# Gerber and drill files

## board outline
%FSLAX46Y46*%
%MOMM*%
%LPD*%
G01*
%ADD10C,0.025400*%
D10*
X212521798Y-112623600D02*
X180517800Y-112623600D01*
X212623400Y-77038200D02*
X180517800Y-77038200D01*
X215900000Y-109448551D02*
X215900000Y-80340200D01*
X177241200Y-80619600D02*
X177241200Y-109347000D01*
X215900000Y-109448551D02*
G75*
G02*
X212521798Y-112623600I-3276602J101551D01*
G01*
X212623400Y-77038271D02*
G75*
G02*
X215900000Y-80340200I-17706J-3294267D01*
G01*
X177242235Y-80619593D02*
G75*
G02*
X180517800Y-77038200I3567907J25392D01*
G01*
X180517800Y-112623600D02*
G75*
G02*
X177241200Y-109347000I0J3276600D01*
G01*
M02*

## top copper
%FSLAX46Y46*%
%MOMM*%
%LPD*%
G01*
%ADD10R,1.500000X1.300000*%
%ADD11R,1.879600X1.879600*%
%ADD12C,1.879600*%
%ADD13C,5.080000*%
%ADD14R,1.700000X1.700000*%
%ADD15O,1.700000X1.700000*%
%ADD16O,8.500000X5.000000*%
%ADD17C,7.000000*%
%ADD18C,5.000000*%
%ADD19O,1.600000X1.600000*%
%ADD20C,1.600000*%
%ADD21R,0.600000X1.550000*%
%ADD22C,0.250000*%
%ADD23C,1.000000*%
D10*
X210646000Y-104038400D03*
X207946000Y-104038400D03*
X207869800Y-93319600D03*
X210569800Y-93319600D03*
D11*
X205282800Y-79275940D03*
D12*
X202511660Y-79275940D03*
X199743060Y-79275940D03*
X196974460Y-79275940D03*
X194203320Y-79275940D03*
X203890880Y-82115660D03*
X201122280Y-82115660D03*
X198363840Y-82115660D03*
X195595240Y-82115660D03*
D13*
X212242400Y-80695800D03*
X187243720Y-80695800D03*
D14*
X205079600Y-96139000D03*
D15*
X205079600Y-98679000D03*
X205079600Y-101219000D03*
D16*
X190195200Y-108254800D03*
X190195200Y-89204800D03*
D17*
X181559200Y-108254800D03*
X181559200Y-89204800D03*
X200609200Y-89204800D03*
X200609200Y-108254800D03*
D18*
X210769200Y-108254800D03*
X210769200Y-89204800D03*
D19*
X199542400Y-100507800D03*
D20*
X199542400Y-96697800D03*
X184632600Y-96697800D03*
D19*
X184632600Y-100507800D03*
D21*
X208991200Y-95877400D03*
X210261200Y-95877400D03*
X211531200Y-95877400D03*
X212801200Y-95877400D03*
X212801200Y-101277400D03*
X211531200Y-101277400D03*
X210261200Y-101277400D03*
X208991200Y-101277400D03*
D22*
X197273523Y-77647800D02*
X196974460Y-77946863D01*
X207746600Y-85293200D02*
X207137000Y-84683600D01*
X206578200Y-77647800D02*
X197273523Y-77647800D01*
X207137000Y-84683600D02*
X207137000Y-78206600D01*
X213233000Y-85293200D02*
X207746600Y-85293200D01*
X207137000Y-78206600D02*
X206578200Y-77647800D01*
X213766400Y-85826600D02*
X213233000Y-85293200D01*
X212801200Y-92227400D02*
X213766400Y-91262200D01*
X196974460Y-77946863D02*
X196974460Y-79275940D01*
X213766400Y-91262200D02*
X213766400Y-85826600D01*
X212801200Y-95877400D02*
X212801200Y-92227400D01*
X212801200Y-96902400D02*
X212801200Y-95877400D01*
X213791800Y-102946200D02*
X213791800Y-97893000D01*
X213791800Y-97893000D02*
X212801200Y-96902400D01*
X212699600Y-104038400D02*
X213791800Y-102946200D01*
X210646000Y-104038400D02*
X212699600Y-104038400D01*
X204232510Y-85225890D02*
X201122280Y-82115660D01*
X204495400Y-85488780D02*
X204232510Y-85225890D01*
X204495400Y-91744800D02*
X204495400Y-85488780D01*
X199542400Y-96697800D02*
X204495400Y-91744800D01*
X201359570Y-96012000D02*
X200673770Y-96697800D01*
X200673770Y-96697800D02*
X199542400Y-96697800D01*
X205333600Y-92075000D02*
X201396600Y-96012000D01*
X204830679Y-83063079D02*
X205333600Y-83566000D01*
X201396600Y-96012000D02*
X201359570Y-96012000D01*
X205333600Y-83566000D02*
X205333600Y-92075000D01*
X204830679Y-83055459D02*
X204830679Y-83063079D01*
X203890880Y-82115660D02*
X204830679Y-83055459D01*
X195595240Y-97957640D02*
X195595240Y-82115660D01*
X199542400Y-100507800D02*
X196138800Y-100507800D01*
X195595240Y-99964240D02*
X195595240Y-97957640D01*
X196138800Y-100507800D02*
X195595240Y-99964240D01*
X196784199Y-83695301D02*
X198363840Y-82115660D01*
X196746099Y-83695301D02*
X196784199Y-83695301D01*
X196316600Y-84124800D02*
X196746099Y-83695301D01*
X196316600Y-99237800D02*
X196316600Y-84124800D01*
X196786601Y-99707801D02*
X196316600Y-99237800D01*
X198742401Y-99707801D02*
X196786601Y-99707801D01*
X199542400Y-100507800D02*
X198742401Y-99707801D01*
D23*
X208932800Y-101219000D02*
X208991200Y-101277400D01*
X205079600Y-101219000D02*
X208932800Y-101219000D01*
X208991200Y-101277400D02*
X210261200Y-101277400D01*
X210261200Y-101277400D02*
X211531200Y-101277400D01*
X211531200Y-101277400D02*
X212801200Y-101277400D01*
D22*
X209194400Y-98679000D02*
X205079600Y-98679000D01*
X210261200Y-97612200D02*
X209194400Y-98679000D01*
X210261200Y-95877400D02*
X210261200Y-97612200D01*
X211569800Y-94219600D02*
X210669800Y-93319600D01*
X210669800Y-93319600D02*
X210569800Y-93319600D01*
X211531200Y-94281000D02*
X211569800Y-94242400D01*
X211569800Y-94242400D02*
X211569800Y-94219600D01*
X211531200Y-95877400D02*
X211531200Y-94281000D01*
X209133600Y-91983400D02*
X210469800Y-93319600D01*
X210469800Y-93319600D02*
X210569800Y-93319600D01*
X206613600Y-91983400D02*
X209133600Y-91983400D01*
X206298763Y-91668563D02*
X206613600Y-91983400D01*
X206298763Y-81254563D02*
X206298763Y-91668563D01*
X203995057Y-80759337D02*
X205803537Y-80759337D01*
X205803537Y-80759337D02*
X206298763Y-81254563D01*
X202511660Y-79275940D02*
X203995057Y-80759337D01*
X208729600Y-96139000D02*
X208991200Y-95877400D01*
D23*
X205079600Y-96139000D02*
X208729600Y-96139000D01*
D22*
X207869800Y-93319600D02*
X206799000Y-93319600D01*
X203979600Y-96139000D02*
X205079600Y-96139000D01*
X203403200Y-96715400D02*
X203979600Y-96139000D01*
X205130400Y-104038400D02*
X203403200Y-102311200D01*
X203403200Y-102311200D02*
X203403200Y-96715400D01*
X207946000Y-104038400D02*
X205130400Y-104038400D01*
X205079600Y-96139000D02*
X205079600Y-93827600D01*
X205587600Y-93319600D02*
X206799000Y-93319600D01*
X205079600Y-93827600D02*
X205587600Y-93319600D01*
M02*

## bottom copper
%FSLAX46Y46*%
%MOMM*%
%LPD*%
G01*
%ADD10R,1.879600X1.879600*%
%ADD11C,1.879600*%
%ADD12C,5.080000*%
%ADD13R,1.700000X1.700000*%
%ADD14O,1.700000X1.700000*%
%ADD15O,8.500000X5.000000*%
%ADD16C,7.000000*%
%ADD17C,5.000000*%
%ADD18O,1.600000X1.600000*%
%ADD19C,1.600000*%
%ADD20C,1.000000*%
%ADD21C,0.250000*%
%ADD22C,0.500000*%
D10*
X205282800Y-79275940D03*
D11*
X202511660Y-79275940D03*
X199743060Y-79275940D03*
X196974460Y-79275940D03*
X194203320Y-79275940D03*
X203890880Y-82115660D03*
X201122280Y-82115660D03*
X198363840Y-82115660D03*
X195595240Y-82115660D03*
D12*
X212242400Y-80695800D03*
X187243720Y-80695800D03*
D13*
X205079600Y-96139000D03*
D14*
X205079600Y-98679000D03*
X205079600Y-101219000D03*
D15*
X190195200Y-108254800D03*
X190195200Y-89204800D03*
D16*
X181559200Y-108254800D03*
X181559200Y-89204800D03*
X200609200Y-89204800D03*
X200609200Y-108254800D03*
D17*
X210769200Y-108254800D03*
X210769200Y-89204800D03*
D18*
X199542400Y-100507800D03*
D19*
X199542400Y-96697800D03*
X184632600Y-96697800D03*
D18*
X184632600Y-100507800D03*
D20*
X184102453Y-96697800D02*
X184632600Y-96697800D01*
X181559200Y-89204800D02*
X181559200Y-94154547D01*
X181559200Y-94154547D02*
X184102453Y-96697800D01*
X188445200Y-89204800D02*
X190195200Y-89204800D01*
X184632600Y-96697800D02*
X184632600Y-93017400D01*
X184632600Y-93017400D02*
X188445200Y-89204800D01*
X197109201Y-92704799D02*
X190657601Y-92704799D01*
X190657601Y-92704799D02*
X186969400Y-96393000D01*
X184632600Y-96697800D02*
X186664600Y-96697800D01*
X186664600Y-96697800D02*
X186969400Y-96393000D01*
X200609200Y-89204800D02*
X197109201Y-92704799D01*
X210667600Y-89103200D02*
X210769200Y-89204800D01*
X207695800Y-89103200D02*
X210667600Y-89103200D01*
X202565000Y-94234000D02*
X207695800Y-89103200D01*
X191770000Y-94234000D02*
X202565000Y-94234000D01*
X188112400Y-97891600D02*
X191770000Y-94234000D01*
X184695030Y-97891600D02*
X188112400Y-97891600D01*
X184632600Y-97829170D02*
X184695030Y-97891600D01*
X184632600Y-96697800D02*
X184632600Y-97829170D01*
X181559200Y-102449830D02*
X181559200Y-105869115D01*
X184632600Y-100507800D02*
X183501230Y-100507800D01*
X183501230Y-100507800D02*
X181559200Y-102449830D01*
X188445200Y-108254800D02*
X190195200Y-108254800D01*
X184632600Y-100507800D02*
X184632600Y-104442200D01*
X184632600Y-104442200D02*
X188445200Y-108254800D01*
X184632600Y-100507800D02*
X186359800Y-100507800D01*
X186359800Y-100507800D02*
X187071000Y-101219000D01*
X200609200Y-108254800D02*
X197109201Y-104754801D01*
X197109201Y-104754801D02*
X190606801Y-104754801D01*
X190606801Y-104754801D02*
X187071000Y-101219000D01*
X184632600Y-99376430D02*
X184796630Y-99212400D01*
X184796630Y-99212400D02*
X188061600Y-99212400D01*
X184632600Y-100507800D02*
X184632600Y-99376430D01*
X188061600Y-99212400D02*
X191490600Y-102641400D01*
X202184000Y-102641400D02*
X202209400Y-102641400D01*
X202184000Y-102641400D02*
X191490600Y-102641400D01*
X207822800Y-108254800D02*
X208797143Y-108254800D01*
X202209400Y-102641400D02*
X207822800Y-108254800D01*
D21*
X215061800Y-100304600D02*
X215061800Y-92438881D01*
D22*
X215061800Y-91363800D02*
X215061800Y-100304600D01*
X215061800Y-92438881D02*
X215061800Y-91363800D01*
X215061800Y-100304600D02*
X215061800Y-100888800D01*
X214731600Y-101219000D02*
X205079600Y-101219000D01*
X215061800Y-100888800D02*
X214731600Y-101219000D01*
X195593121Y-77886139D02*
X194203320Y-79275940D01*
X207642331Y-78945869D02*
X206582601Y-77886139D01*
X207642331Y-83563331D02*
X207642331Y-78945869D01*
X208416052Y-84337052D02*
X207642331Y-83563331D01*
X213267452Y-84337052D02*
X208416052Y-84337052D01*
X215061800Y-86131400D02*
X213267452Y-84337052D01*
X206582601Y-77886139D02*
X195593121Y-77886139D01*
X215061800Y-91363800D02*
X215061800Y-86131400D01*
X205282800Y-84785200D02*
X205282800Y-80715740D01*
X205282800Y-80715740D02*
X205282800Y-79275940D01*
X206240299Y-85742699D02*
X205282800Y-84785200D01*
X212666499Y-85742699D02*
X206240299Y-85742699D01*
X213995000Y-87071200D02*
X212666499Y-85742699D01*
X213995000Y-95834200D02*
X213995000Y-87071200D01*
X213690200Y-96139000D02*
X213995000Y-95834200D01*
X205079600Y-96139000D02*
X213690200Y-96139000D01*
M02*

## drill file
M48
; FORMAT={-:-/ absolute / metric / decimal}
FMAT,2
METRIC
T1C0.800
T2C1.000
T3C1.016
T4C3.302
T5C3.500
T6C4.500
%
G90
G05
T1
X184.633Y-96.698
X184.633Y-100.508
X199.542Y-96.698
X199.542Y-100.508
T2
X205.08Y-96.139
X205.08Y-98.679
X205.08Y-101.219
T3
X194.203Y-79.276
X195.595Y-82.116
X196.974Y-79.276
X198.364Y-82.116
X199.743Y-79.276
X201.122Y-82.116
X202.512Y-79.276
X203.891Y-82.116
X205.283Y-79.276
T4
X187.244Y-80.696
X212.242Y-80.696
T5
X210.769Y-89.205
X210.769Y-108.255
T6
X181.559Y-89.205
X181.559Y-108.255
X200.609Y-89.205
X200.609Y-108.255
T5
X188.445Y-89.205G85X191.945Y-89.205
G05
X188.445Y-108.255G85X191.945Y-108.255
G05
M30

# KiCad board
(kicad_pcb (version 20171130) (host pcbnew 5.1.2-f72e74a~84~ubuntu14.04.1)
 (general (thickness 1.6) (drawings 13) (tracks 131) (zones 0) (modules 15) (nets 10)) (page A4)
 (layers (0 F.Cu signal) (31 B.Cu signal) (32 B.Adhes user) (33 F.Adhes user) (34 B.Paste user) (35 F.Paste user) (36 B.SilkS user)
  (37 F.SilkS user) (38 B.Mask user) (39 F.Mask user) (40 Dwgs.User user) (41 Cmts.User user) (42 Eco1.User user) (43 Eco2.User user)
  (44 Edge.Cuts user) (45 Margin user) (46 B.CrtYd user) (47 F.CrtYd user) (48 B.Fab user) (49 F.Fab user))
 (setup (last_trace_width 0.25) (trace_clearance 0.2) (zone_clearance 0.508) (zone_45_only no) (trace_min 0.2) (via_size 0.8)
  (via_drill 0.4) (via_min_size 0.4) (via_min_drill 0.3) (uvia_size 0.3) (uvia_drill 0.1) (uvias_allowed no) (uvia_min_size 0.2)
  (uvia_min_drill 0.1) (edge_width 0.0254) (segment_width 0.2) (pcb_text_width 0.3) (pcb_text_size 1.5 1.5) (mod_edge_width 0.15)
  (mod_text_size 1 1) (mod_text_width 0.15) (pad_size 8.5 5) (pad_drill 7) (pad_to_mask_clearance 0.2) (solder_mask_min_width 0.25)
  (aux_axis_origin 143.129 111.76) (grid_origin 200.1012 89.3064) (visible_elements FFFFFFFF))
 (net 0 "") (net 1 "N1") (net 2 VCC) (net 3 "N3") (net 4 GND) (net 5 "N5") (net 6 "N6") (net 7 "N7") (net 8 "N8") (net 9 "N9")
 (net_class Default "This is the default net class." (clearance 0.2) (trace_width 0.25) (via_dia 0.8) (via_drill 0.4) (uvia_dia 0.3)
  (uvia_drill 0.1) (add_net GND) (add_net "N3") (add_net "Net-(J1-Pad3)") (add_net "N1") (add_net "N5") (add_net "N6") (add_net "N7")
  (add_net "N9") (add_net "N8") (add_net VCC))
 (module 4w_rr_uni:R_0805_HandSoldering (layer F.Cu) (at 209.296 104.0384)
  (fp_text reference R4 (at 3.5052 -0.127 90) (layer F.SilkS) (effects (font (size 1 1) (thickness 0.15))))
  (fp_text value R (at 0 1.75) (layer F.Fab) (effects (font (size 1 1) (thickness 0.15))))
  (pad 2 smd rect (at 1.35 0) (size 1.5 1.3) (layers F.Cu F.Paste F.Mask) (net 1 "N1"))
  (pad 1 smd rect (at -1.35 0) (size 1.5 1.3) (layers F.Cu F.Paste F.Mask) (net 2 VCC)))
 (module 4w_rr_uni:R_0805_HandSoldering (layer F.Cu) (at 209.2198 93.3196)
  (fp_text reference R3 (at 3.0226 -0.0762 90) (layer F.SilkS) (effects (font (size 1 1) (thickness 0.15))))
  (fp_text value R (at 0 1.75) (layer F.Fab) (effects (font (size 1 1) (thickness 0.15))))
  (pad 1 smd rect (at -1.35 0) (size 1.5 1.3) (layers F.Cu F.Paste F.Mask) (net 2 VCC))
  (pad 2 smd rect (at 1.35 0) (size 1.5 1.3) (layers F.Cu F.Paste F.Mask) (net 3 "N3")))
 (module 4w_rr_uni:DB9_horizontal (layer F.Cu) (at 199.74306 80.6958 180)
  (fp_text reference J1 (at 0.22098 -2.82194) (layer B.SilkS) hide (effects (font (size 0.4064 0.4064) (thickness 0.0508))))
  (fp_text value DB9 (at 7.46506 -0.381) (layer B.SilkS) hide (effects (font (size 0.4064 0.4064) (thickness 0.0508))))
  (pad 1 thru_hole rect (at -5.53974 1.41986 180) (size 1.8796 1.8796) (drill 1.016) (layers F&B.Cu F.Paste F.SilkS F.Mask) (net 2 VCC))
  (pad 2 thru_hole circle (at -2.7686 1.41986 180) (size 1.8796 1.8796) (drill 1.016) (layers F&B.Cu F.Paste F.SilkS F.Mask) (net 3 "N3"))
  (pad 3 thru_hole circle (at 0 1.41986 180) (size 1.8796 1.8796) (drill 1.016) (layers F&B.Cu F.Paste F.SilkS F.Mask))
  (pad 4 thru_hole circle (at 2.7686 1.41986 180) (size 1.8796 1.8796) (drill 1.016) (layers F&B.Cu F.Paste F.SilkS F.Mask) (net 1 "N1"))
  (pad 5 thru_hole circle (at 5.53974 1.41986 180) (size 1.8796 1.8796) (drill 1.016) (layers F&B.Cu F.Paste F.SilkS F.Mask) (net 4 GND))
  (pad 6 thru_hole circle (at -4.14782 -1.41986 180) (size 1.8796 1.8796) (drill 1.016) (layers F&B.Cu F.Paste F.SilkS F.Mask) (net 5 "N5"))
  (pad 7 thru_hole circle (at -1.37922 -1.41986 180) (size 1.8796 1.8796) (drill 1.016) (layers F&B.Cu F.Paste F.SilkS F.Mask) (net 5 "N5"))
  (pad 8 thru_hole circle (at 1.37922 -1.41986 180) (size 1.8796 1.8796) (drill 1.016) (layers F&B.Cu F.Paste F.SilkS F.Mask) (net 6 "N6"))
  (pad 9 thru_hole circle (at 4.14782 -1.41986 180) (size 1.8796 1.8796) (drill 1.016) (layers F&B.Cu F.Paste F.SilkS F.Mask) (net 6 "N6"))
  (pad G1 thru_hole circle (at -12.49934 0 180) (size 5.08 5.08) (drill 3.302) (layers F&B.Cu F.Paste F.SilkS F.Mask))
  (pad G2 thru_hole circle (at 12.49934 0 180) (size 5.08 5.08) (drill 3.302) (layers F&B.Cu F.Paste F.SilkS F.Mask)))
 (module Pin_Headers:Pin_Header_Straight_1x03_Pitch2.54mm (layer F.Cu) (at 205.0796 96.139)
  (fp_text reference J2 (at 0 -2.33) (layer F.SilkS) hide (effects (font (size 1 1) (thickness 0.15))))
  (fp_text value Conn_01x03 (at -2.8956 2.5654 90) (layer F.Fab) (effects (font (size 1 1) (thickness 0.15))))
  (pad 1 thru_hole rect (at 0 0) (size 1.7 1.7) (drill 1) (layers *.Cu *.Mask) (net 2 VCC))
  (pad 2 thru_hole oval (at 0 2.54) (size 1.7 1.7) (drill 1) (layers *.Cu *.Mask) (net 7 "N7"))
  (pad 3 thru_hole oval (at 0 5.08) (size 1.7 1.7) (drill 1) (layers *.Cu *.Mask) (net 4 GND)))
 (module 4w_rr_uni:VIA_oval (layer F.Cu) (at 190.4492 108.2548)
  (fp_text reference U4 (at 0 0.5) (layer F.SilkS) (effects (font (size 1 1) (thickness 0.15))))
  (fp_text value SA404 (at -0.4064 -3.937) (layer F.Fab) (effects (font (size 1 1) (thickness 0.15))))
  (pad 1 thru_hole oval (at -0.254 0) (size 8.5 5) (drill oval 7 3.5) (layers *.Cu *.Mask) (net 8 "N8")))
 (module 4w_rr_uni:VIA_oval (layer F.Cu) (at 190.4492 89.2048)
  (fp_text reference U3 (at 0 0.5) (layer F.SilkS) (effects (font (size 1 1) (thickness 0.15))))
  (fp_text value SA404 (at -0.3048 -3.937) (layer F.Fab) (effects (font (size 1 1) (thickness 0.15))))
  (pad 1 thru_hole oval (at -0.254 0) (size 8.5 5) (drill oval 7 3.5) (layers *.Cu *.Mask) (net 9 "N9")))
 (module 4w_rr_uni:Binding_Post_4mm (layer F.Cu) (at 181.5592 108.2548)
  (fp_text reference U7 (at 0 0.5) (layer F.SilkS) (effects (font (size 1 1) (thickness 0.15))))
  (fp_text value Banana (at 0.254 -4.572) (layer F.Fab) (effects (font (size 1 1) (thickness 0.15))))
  (pad 1 thru_hole circle (at 0 0) (size 7 7) (drill 4.5) (layers *.Cu *.Mask) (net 8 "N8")))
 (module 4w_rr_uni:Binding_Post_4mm (layer F.Cu) (at 181.5592 89.2048)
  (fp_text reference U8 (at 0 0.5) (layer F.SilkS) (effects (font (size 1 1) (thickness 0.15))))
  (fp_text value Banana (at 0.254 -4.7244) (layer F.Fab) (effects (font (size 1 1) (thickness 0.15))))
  (pad 1 thru_hole circle (at 0 0) (size 7 7) (drill 4.5) (layers *.Cu *.Mask) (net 9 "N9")))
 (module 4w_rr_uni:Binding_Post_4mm (layer F.Cu) (at 200.6092 89.2048)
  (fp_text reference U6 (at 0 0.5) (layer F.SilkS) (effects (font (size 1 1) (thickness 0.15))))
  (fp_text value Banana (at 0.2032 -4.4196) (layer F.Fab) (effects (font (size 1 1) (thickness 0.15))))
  (pad 1 thru_hole circle (at 0 0) (size 7 7) (drill 4.5) (layers *.Cu *.Mask) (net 9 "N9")))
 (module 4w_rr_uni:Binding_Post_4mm (layer F.Cu) (at 200.6092 108.2548)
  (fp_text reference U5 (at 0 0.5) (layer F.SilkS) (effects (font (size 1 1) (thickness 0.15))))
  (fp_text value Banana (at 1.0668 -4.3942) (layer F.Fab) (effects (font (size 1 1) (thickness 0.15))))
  (pad 1 thru_hole circle (at 0 0) (size 7 7) (drill 4.5) (layers *.Cu *.Mask) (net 8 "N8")))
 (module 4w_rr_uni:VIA (layer F.Cu) (at 210.7692 108.2548)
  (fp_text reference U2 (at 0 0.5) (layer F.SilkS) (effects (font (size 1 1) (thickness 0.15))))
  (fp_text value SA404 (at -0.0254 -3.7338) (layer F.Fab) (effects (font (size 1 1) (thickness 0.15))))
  (pad 1 thru_hole circle (at 0 0) (size 5 5) (drill 3.5) (layers *.Cu *.Mask) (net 8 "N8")))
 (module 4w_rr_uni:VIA (layer F.Cu) (at 210.7692 89.2048)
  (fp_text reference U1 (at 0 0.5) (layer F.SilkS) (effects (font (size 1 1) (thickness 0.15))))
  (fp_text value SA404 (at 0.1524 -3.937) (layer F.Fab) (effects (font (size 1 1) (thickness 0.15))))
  (pad 1 thru_hole circle (at 0 0) (size 5 5) (drill 3.5) (layers *.Cu *.Mask) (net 9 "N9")))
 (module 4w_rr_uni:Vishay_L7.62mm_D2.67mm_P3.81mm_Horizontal (layer F.Cu) (at 199.5424 98.6028 270)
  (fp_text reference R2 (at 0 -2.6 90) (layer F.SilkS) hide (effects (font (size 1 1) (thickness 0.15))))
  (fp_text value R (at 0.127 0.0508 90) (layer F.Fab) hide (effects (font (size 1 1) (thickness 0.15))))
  (pad 2 thru_hole oval (at 1.905 0 270) (size 1.6 1.6) (drill 0.8) (layers *.Cu *.Mask) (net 6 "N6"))
  (pad 1 thru_hole circle (at -1.905 0 270) (size 1.6 1.6) (drill 0.8) (layers *.Cu *.Mask) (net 5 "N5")))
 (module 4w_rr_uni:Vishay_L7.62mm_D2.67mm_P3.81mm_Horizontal (layer F.Cu) (at 184.6326 98.6028 270)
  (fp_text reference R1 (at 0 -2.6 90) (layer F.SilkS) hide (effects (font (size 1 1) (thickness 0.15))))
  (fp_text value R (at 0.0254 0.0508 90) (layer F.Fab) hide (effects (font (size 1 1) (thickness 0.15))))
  (pad 1 thru_hole circle (at -1.905 0 270) (size 1.6 1.6) (drill 0.8) (layers *.Cu *.Mask) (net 9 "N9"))
  (pad 2 thru_hole oval (at 1.905 0 270) (size 1.6 1.6) (drill 0.8) (layers *.Cu *.Mask) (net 8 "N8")))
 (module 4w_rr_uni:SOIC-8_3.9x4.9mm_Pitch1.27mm (layer F.Cu) (at 210.8962 98.5774 90)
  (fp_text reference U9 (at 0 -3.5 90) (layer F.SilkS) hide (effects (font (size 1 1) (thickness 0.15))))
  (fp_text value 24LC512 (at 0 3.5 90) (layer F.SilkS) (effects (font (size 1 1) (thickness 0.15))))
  (pad 8 smd rect (at 2.7 -1.905 90) (size 1.55 0.6) (layers F.Cu F.Paste F.Mask) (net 2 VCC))
  (pad 7 smd rect (at 2.7 -0.635 90) (size 1.55 0.6) (layers F.Cu F.Paste F.Mask) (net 7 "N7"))
  (pad 6 smd rect (at 2.7 0.635 90) (size 1.55 0.6) (layers F.Cu F.Paste F.Mask) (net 3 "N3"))
  (pad 5 smd rect (at 2.7 1.905 90) (size 1.55 0.6) (layers F.Cu F.Paste F.Mask) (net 1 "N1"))
  (pad 4 smd rect (at -2.7 1.905 90) (size 1.55 0.6) (layers F.Cu F.Paste F.Mask) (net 4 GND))
  (pad 3 smd rect (at -2.7 0.635 90) (size 1.55 0.6) (layers F.Cu F.Paste F.Mask) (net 4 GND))
  (pad 2 smd rect (at -2.7 -0.635 90) (size 1.55 0.6) (layers F.Cu F.Paste F.Mask) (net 4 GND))
  (pad 1 smd rect (at -2.7 -1.905 90) (size 1.55 0.6) (layers F.Cu F.Paste F.Mask) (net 4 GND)))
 (gr_line (start 212.521798 112.6236) (end 180.5178 112.6236) (layer Edge.Cuts) (width 0.0254))
 (gr_line (start 212.6234 77.0382) (end 180.5178 77.0382) (layer Edge.Cuts) (width 0.0254))
 (gr_line (start 215.9 109.448551) (end 215.9 80.3402) (layer Edge.Cuts) (width 0.0254))
 (gr_line (start 177.2412 80.6196) (end 177.2412 109.347) (layer Edge.Cuts) (width 0.0254))
 (gr_arc (start 212.623398 109.347) (end 212.521798 112.6236) (angle -90.00085275) (layer Edge.Cuts) (width 0.0254))
 (gr_arc (start 212.605694 80.332538) (end 215.9 80.3402) (angle -89.82531014) (layer Edge.Cuts) (width 0.0254))
 (gr_arc (start 180.810142 80.594201) (end 180.5178 77.0382) (angle -85.7079865) (layer Edge.Cuts) (width 0.0254))
 (gr_arc (start 180.5178 109.347) (end 177.2412 109.347) (angle -90) (layer Edge.Cuts) (width 0.0254))
 (segment (start 184.102453 96.6978) (end 184.6326 96.6978) (width 1) (layer B.Cu) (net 9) (status 30))
 (segment (start 181.5592 89.2048) (end 181.5592 94.154547) (width 1) (layer B.Cu) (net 9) (status 10))
 (segment (start 181.5592 94.154547) (end 184.102453 96.6978) (width 1) (layer B.Cu) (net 9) (status 20))
 (segment (start 188.4452 89.2048) (end 190.1952 89.2048) (width 1) (layer B.Cu) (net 9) (status 30))
 (segment (start 184.6326 96.6978) (end 184.6326 93.0174) (width 1) (layer B.Cu) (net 9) (status 10))
 (segment (start 184.6326 93.0174) (end 188.4452 89.2048) (width 1) (layer B.Cu) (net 9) (status 20))
 (segment (start 197.109201 92.704799) (end 190.657601 92.704799) (width 1) (layer B.Cu) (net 9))
 (segment (start 190.657601 92.704799) (end 186.9694 96.393) (width 1) (layer B.Cu) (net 9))
 (segment (start 184.6326 96.6978) (end 186.6646 96.6978) (width 1) (layer B.Cu) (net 9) (status 10))
 (segment (start 186.6646 96.6978) (end 186.9694 96.393) (width 1) (layer B.Cu) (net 9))
 (segment (start 200.6092 89.2048) (end 197.109201 92.704799) (width 1) (layer B.Cu) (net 9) (status 10))
 (segment (start 210.6676 89.1032) (end 210.7692 89.2048) (width 1) (layer B.Cu) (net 9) (status 30))
 (segment (start 207.6958 89.1032) (end 210.6676 89.1032) (width 1) (layer B.Cu) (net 9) (status 20))
 (segment (start 202.565 94.234) (end 207.6958 89.1032) (width 1) (layer B.Cu) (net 9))
 (segment (start 191.77 94.234) (end 202.565 94.234) (width 1) (layer B.Cu) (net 9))
 (segment (start 188.1124 97.8916) (end 191.77 94.234) (width 1) (layer B.Cu) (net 9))
 (segment (start 184.69503 97.8916) (end 188.1124 97.8916) (width 1) (layer B.Cu) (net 9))
 (segment (start 184.6326 97.82917) (end 184.69503 97.8916) (width 1) (layer B.Cu) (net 9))
 (segment (start 184.6326 96.6978) (end 184.6326 97.82917) (width 1) (layer B.Cu) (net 9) (status 10))
 (segment (start 181.5592 102.44983) (end 181.5592 105.869115) (width 1) (layer B.Cu) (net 8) (status 20))
 (segment (start 184.6326 100.5078) (end 183.50123 100.5078) (width 1) (layer B.Cu) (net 8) (status 10))
 (segment (start 183.50123 100.5078) (end 181.5592 102.44983) (width 1) (layer B.Cu) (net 8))
 (segment (start 188.4452 108.2548) (end 190.1952 108.2548) (width 1) (layer B.Cu) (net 8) (status 30))
 (segment (start 184.6326 100.5078) (end 184.6326 104.4422) (width 1) (layer B.Cu) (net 8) (status 10))
 (segment (start 184.6326 104.4422) (end 188.4452 108.2548) (width 1) (layer B.Cu) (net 8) (status 20))
 (segment (start 184.6326 100.5078) (end 186.3598 100.5078) (width 1) (layer B.Cu) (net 8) (status 10))
 (segment (start 186.3598 100.5078) (end 187.071 101.219) (width 1) (layer B.Cu) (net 8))
 (segment (start 200.6092 108.2548) (end 197.109201 104.754801) (width 1) (layer B.Cu) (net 8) (status 10))
 (segment (start 197.109201 104.754801) (end 190.606801 104.754801) (width 1) (layer B.Cu) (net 8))
 (segment (start 190.606801 104.754801) (end 187.071 101.219) (width 1) (layer B.Cu) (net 8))
 (segment (start 184.6326 99.37643) (end 184.79663 99.2124) (width 1) (layer B.Cu) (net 8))
 (segment (start 184.79663 99.2124) (end 188.0616 99.2124) (width 1) (layer B.Cu) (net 8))
 (segment (start 184.6326 100.5078) (end 184.6326 99.37643) (width 1) (layer B.Cu) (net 8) (status 10))
 (segment (start 188.0616 99.2124) (end 191.4906 102.6414) (width 1) (layer B.Cu) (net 8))
 (segment (start 202.184 102.6414) (end 202.2094 102.6414) (width 1) (layer B.Cu) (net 8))
 (segment (start 202.184 102.6414) (end 191.4906 102.6414) (width 1) (layer B.Cu) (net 8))
 (segment (start 207.8228 108.2548) (end 208.797143 108.2548) (width 1) (layer B.Cu) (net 8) (status 20))
 (segment (start 202.2094 102.6414) (end 207.8228 108.2548) (width 1) (layer B.Cu) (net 8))
 (segment (start 197.273523 77.6478) (end 196.97446 77.946863) (width 0.25) (layer F.Cu) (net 1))
 (segment (start 207.7466 85.2932) (end 207.137 84.6836) (width 0.25) (layer F.Cu) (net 1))
 (segment (start 206.5782 77.6478) (end 197.273523 77.6478) (width 0.25) (layer F.Cu) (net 1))
 (segment (start 207.137 84.6836) (end 207.137 78.2066) (width 0.25) (layer F.Cu) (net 1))
 (segment (start 213.233 85.2932) (end 207.7466 85.2932) (width 0.25) (layer F.Cu) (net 1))
 (segment (start 207.137 78.2066) (end 206.5782 77.6478) (width 0.25) (layer F.Cu) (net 1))
 (segment (start 213.7664 85.8266) (end 213.233 85.2932) (width 0.25) (layer F.Cu) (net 1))
 (segment (start 212.8012 92.2274) (end 213.7664 91.2622) (width 0.25) (layer F.Cu) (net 1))
 (segment (start 196.97446 77.946863) (end 196.97446 79.27594) (width 0.25) (layer F.Cu) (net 1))
 (segment (start 213.7664 91.2622) (end 213.7664 85.8266) (width 0.25) (layer F.Cu) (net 1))
 (segment (start 212.8012 95.8774) (end 212.8012 92.2274) (width 0.25) (layer F.Cu) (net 1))
 (segment (start 212.8012 96.9024) (end 212.8012 95.8774) (width 0.25) (layer F.Cu) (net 1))
 (segment (start 213.7918 102.9462) (end 213.7918 97.893) (width 0.25) (layer F.Cu) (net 1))
 (segment (start 213.7918 97.893) (end 212.8012 96.9024) (width 0.25) (layer F.Cu) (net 1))
 (segment (start 212.6996 104.0384) (end 213.7918 102.9462) (width 0.25) (layer F.Cu) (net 1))
 (segment (start 210.646 104.0384) (end 212.6996 104.0384) (width 0.25) (layer F.Cu) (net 1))
 (segment (start 204.23251 85.22589) (end 201.12228 82.11566) (width 0.25) (layer F.Cu) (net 5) (status 20))
 (segment (start 204.4954 85.48878) (end 204.23251 85.22589) (width 0.25) (layer F.Cu) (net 5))
 (segment (start 204.4954 91.7448) (end 204.4954 85.48878) (width 0.25) (layer F.Cu) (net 5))
 (segment (start 199.5424 96.6978) (end 204.4954 91.7448) (width 0.25) (layer F.Cu) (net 5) (status 10))
 (segment (start 201.35957 96.012) (end 200.67377 96.6978) (width 0.25) (layer F.Cu) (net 5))
 (segment (start 200.67377 96.6978) (end 199.5424 96.6978) (width 0.25) (layer F.Cu) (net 5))
 (segment (start 205.3336 92.075) (end 201.3966 96.012) (width 0.25) (layer F.Cu) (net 5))
 (segment (start 204.830679 83.063079) (end 205.3336 83.566) (width 0.25) (layer F.Cu) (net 5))
 (segment (start 201.3966 96.012) (end 201.35957 96.012) (width 0.25) (layer F.Cu) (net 5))
 (segment (start 205.3336 83.566) (end 205.3336 92.075) (width 0.25) (layer F.Cu) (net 5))
 (segment (start 204.830679 83.055459) (end 204.830679 83.063079) (width 0.25) (layer F.Cu) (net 5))
 (segment (start 203.89088 82.11566) (end 204.830679 83.055459) (width 0.25) (layer F.Cu) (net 5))
 (segment (start 195.59524 97.95764) (end 195.59524 82.11566) (width 0.25) (layer F.Cu) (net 6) (status 20))
 (segment (start 199.5424 100.5078) (end 196.1388 100.5078) (width 0.25) (layer F.Cu) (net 6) (status 10))
 (segment (start 195.59524 99.96424) (end 195.59524 97.95764) (width 0.25) (layer F.Cu) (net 6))
 (segment (start 196.1388 100.5078) (end 195.59524 99.96424) (width 0.25) (layer F.Cu) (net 6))
 (segment (start 196.784199 83.695301) (end 198.36384 82.11566) (width 0.25) (layer F.Cu) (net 6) (status 20))
 (segment (start 196.746099 83.695301) (end 196.784199 83.695301) (width 0.25) (layer F.Cu) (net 6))
 (segment (start 196.3166 84.1248) (end 196.746099 83.695301) (width 0.25) (layer F.Cu) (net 6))
 (segment (start 196.3166 99.2378) (end 196.3166 84.1248) (width 0.25) (layer F.Cu) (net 6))
 (segment (start 196.786601 99.707801) (end 196.3166 99.2378) (width 0.25) (layer F.Cu) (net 6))
 (segment (start 198.742401 99.707801) (end 196.786601 99.707801) (width 0.25) (layer F.Cu) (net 6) (status 10))
 (segment (start 199.5424 100.5078) (end 198.742401 99.707801) (width 0.25) (layer F.Cu) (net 6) (status 30))
 (segment (start 215.0618 100.3046) (end 215.0618 92.438881) (width 0.25) (layer B.Cu) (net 4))
 (segment (start 215.0618 91.3638) (end 215.0618 100.3046) (width 0.5) (layer B.Cu) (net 4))
 (segment (start 215.0618 92.438881) (end 215.0618 91.3638) (width 0.5) (layer B.Cu) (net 4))
 (segment (start 208.9328 101.219) (end 208.9912 101.2774) (width 1) (layer F.Cu) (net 4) (status 30))
 (segment (start 205.0796 101.219) (end 208.9328 101.219) (width 1) (layer F.Cu) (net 4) (status 30))
 (segment (start 215.0618 100.3046) (end 215.0618 100.8888) (width 0.5) (layer B.Cu) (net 4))
 (segment (start 214.7316 101.219) (end 205.0796 101.219) (width 0.5) (layer B.Cu) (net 4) (status 20))
 (segment (start 215.0618 100.8888) (end 214.7316 101.219) (width 0.5) (layer B.Cu) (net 4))
 (segment (start 208.9912 101.2774) (end 210.2612 101.2774) (width 1) (layer F.Cu) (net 4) (status 30))
 (segment (start 210.2612 101.2774) (end 211.5312 101.2774) (width 1) (layer F.Cu) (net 4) (status 30))
 (segment (start 211.5312 101.2774) (end 212.8012 101.2774) (width 1) (layer F.Cu) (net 4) (status 30))
 (segment (start 195.593121 77.886139) (end 194.20332 79.27594) (width 0.5) (layer B.Cu) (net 4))
 (segment (start 207.642331 78.945869) (end 206.582601 77.886139) (width 0.5) (layer B.Cu) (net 4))
 (segment (start 207.642331 83.563331) (end 207.642331 78.945869) (width 0.5) (layer B.Cu) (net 4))
 (segment (start 208.416052 84.337052) (end 207.642331 83.563331) (width 0.5) (layer B.Cu) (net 4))
 (segment (start 213.267452 84.337052) (end 208.416052 84.337052) (width 0.5) (layer B.Cu) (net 4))
 (segment (start 215.0618 86.1314) (end 213.267452 84.337052) (width 0.5) (layer B.Cu) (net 4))
 (segment (start 206.582601 77.886139) (end 195.593121 77.886139) (width 0.5) (layer B.Cu) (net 4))
 (segment (start 215.0618 91.3638) (end 215.0618 86.1314) (width 0.5) (layer B.Cu) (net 4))
 (segment (start 209.1944 98.679) (end 205.0796 98.679) (width 0.25) (layer F.Cu) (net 7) (status 20))
 (segment (start 210.2612 97.6122) (end 209.1944 98.679) (width 0.25) (layer F.Cu) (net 7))
 (segment (start 210.2612 95.8774) (end 210.2612 97.6122) (width 0.25) (layer F.Cu) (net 7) (status 10))
 (segment (start 211.5698 94.2196) (end 210.6698 93.3196) (width 0.25) (layer F.Cu) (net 3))
 (segment (start 210.6698 93.3196) (end 210.5698 93.3196) (width 0.25) (layer F.Cu) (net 3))
 (segment (start 211.5312 94.281) (end 211.5698 94.2424) (width 0.25) (layer F.Cu) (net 3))
 (segment (start 211.5698 94.2424) (end 211.5698 94.2196) (width 0.25) (layer F.Cu) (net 3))
 (segment (start 211.5312 95.8774) (end 211.5312 94.281) (width 0.25) (layer F.Cu) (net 3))
 (segment (start 209.1336 91.9834) (end 210.4698 93.3196) (width 0.25) (layer F.Cu) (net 3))
 (segment (start 210.4698 93.3196) (end 210.5698 93.3196) (width 0.25) (layer F.Cu) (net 3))
 (segment (start 206.6136 91.9834) (end 209.1336 91.9834) (width 0.25) (layer F.Cu) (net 3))
 (segment (start 206.298763 91.668563) (end 206.6136 91.9834) (width 0.25) (layer F.Cu) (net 3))
 (segment (start 206.298763 81.254563) (end 206.298763 91.668563) (width 0.25) (layer F.Cu) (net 3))
 (segment (start 203.995057 80.759337) (end 205.803537 80.759337) (width 0.25) (layer F.Cu) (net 3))
 (segment (start 205.803537 80.759337) (end 206.298763 81.254563) (width 0.25) (layer F.Cu) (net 3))
 (segment (start 202.51166 79.27594) (end 203.995057 80.759337) (width 0.25) (layer F.Cu) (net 3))
 (segment (start 208.7296 96.139) (end 208.9912 95.8774) (width 0.25) (layer F.Cu) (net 2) (status 30))
 (segment (start 205.0796 96.139) (end 208.7296 96.139) (width 1) (layer F.Cu) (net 2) (status 30))
 (segment (start 205.2828 84.7852) (end 205.2828 80.71574) (width 0.5) (layer B.Cu) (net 2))
 (segment (start 205.2828 80.71574) (end 205.2828 79.27594) (width 0.5) (layer B.Cu) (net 2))
 (segment (start 206.240299 85.742699) (end 205.2828 84.7852) (width 0.5) (layer B.Cu) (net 2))
 (segment (start 212.666499 85.742699) (end 206.240299 85.742699) (width 0.5) (layer B.Cu) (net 2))
 (segment (start 213.995 87.0712) (end 212.666499 85.742699) (width 0.5) (layer B.Cu) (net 2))
 (segment (start 213.995 95.8342) (end 213.995 87.0712) (width 0.5) (layer B.Cu) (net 2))
 (segment (start 213.6902 96.139) (end 213.995 95.8342) (width 0.5) (layer B.Cu) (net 2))
 (segment (start 205.0796 96.139) (end 213.6902 96.139) (width 0.5) (layer B.Cu) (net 2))
 (segment (start 207.8698 93.3196) (end 206.799 93.3196) (width 0.25) (layer F.Cu) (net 2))
 (segment (start 203.9796 96.139) (end 205.0796 96.139) (width 0.25) (layer F.Cu) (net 2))
 (segment (start 203.4032 96.7154) (end 203.9796 96.139) (width 0.25) (layer F.Cu) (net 2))
 (segment (start 205.1304 104.0384) (end 203.4032 102.3112) (width 0.25) (layer F.Cu) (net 2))
 (segment (start 203.4032 102.3112) (end 203.4032 96.7154) (width 0.25) (layer F.Cu) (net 2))
 (segment (start 207.946 104.0384) (end 205.1304 104.0384) (width 0.25) (layer F.Cu) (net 2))
 (segment (start 205.0796 96.139) (end 205.0796 93.8276) (width 0.25) (layer F.Cu) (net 2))
 (segment (start 205.5876 93.3196) (end 206.799 93.3196) (width 0.25) (layer F.Cu) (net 2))
 (segment (start 205.0796 93.8276) (end 205.5876 93.3196) (width 0.25) (layer F.Cu) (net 2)))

